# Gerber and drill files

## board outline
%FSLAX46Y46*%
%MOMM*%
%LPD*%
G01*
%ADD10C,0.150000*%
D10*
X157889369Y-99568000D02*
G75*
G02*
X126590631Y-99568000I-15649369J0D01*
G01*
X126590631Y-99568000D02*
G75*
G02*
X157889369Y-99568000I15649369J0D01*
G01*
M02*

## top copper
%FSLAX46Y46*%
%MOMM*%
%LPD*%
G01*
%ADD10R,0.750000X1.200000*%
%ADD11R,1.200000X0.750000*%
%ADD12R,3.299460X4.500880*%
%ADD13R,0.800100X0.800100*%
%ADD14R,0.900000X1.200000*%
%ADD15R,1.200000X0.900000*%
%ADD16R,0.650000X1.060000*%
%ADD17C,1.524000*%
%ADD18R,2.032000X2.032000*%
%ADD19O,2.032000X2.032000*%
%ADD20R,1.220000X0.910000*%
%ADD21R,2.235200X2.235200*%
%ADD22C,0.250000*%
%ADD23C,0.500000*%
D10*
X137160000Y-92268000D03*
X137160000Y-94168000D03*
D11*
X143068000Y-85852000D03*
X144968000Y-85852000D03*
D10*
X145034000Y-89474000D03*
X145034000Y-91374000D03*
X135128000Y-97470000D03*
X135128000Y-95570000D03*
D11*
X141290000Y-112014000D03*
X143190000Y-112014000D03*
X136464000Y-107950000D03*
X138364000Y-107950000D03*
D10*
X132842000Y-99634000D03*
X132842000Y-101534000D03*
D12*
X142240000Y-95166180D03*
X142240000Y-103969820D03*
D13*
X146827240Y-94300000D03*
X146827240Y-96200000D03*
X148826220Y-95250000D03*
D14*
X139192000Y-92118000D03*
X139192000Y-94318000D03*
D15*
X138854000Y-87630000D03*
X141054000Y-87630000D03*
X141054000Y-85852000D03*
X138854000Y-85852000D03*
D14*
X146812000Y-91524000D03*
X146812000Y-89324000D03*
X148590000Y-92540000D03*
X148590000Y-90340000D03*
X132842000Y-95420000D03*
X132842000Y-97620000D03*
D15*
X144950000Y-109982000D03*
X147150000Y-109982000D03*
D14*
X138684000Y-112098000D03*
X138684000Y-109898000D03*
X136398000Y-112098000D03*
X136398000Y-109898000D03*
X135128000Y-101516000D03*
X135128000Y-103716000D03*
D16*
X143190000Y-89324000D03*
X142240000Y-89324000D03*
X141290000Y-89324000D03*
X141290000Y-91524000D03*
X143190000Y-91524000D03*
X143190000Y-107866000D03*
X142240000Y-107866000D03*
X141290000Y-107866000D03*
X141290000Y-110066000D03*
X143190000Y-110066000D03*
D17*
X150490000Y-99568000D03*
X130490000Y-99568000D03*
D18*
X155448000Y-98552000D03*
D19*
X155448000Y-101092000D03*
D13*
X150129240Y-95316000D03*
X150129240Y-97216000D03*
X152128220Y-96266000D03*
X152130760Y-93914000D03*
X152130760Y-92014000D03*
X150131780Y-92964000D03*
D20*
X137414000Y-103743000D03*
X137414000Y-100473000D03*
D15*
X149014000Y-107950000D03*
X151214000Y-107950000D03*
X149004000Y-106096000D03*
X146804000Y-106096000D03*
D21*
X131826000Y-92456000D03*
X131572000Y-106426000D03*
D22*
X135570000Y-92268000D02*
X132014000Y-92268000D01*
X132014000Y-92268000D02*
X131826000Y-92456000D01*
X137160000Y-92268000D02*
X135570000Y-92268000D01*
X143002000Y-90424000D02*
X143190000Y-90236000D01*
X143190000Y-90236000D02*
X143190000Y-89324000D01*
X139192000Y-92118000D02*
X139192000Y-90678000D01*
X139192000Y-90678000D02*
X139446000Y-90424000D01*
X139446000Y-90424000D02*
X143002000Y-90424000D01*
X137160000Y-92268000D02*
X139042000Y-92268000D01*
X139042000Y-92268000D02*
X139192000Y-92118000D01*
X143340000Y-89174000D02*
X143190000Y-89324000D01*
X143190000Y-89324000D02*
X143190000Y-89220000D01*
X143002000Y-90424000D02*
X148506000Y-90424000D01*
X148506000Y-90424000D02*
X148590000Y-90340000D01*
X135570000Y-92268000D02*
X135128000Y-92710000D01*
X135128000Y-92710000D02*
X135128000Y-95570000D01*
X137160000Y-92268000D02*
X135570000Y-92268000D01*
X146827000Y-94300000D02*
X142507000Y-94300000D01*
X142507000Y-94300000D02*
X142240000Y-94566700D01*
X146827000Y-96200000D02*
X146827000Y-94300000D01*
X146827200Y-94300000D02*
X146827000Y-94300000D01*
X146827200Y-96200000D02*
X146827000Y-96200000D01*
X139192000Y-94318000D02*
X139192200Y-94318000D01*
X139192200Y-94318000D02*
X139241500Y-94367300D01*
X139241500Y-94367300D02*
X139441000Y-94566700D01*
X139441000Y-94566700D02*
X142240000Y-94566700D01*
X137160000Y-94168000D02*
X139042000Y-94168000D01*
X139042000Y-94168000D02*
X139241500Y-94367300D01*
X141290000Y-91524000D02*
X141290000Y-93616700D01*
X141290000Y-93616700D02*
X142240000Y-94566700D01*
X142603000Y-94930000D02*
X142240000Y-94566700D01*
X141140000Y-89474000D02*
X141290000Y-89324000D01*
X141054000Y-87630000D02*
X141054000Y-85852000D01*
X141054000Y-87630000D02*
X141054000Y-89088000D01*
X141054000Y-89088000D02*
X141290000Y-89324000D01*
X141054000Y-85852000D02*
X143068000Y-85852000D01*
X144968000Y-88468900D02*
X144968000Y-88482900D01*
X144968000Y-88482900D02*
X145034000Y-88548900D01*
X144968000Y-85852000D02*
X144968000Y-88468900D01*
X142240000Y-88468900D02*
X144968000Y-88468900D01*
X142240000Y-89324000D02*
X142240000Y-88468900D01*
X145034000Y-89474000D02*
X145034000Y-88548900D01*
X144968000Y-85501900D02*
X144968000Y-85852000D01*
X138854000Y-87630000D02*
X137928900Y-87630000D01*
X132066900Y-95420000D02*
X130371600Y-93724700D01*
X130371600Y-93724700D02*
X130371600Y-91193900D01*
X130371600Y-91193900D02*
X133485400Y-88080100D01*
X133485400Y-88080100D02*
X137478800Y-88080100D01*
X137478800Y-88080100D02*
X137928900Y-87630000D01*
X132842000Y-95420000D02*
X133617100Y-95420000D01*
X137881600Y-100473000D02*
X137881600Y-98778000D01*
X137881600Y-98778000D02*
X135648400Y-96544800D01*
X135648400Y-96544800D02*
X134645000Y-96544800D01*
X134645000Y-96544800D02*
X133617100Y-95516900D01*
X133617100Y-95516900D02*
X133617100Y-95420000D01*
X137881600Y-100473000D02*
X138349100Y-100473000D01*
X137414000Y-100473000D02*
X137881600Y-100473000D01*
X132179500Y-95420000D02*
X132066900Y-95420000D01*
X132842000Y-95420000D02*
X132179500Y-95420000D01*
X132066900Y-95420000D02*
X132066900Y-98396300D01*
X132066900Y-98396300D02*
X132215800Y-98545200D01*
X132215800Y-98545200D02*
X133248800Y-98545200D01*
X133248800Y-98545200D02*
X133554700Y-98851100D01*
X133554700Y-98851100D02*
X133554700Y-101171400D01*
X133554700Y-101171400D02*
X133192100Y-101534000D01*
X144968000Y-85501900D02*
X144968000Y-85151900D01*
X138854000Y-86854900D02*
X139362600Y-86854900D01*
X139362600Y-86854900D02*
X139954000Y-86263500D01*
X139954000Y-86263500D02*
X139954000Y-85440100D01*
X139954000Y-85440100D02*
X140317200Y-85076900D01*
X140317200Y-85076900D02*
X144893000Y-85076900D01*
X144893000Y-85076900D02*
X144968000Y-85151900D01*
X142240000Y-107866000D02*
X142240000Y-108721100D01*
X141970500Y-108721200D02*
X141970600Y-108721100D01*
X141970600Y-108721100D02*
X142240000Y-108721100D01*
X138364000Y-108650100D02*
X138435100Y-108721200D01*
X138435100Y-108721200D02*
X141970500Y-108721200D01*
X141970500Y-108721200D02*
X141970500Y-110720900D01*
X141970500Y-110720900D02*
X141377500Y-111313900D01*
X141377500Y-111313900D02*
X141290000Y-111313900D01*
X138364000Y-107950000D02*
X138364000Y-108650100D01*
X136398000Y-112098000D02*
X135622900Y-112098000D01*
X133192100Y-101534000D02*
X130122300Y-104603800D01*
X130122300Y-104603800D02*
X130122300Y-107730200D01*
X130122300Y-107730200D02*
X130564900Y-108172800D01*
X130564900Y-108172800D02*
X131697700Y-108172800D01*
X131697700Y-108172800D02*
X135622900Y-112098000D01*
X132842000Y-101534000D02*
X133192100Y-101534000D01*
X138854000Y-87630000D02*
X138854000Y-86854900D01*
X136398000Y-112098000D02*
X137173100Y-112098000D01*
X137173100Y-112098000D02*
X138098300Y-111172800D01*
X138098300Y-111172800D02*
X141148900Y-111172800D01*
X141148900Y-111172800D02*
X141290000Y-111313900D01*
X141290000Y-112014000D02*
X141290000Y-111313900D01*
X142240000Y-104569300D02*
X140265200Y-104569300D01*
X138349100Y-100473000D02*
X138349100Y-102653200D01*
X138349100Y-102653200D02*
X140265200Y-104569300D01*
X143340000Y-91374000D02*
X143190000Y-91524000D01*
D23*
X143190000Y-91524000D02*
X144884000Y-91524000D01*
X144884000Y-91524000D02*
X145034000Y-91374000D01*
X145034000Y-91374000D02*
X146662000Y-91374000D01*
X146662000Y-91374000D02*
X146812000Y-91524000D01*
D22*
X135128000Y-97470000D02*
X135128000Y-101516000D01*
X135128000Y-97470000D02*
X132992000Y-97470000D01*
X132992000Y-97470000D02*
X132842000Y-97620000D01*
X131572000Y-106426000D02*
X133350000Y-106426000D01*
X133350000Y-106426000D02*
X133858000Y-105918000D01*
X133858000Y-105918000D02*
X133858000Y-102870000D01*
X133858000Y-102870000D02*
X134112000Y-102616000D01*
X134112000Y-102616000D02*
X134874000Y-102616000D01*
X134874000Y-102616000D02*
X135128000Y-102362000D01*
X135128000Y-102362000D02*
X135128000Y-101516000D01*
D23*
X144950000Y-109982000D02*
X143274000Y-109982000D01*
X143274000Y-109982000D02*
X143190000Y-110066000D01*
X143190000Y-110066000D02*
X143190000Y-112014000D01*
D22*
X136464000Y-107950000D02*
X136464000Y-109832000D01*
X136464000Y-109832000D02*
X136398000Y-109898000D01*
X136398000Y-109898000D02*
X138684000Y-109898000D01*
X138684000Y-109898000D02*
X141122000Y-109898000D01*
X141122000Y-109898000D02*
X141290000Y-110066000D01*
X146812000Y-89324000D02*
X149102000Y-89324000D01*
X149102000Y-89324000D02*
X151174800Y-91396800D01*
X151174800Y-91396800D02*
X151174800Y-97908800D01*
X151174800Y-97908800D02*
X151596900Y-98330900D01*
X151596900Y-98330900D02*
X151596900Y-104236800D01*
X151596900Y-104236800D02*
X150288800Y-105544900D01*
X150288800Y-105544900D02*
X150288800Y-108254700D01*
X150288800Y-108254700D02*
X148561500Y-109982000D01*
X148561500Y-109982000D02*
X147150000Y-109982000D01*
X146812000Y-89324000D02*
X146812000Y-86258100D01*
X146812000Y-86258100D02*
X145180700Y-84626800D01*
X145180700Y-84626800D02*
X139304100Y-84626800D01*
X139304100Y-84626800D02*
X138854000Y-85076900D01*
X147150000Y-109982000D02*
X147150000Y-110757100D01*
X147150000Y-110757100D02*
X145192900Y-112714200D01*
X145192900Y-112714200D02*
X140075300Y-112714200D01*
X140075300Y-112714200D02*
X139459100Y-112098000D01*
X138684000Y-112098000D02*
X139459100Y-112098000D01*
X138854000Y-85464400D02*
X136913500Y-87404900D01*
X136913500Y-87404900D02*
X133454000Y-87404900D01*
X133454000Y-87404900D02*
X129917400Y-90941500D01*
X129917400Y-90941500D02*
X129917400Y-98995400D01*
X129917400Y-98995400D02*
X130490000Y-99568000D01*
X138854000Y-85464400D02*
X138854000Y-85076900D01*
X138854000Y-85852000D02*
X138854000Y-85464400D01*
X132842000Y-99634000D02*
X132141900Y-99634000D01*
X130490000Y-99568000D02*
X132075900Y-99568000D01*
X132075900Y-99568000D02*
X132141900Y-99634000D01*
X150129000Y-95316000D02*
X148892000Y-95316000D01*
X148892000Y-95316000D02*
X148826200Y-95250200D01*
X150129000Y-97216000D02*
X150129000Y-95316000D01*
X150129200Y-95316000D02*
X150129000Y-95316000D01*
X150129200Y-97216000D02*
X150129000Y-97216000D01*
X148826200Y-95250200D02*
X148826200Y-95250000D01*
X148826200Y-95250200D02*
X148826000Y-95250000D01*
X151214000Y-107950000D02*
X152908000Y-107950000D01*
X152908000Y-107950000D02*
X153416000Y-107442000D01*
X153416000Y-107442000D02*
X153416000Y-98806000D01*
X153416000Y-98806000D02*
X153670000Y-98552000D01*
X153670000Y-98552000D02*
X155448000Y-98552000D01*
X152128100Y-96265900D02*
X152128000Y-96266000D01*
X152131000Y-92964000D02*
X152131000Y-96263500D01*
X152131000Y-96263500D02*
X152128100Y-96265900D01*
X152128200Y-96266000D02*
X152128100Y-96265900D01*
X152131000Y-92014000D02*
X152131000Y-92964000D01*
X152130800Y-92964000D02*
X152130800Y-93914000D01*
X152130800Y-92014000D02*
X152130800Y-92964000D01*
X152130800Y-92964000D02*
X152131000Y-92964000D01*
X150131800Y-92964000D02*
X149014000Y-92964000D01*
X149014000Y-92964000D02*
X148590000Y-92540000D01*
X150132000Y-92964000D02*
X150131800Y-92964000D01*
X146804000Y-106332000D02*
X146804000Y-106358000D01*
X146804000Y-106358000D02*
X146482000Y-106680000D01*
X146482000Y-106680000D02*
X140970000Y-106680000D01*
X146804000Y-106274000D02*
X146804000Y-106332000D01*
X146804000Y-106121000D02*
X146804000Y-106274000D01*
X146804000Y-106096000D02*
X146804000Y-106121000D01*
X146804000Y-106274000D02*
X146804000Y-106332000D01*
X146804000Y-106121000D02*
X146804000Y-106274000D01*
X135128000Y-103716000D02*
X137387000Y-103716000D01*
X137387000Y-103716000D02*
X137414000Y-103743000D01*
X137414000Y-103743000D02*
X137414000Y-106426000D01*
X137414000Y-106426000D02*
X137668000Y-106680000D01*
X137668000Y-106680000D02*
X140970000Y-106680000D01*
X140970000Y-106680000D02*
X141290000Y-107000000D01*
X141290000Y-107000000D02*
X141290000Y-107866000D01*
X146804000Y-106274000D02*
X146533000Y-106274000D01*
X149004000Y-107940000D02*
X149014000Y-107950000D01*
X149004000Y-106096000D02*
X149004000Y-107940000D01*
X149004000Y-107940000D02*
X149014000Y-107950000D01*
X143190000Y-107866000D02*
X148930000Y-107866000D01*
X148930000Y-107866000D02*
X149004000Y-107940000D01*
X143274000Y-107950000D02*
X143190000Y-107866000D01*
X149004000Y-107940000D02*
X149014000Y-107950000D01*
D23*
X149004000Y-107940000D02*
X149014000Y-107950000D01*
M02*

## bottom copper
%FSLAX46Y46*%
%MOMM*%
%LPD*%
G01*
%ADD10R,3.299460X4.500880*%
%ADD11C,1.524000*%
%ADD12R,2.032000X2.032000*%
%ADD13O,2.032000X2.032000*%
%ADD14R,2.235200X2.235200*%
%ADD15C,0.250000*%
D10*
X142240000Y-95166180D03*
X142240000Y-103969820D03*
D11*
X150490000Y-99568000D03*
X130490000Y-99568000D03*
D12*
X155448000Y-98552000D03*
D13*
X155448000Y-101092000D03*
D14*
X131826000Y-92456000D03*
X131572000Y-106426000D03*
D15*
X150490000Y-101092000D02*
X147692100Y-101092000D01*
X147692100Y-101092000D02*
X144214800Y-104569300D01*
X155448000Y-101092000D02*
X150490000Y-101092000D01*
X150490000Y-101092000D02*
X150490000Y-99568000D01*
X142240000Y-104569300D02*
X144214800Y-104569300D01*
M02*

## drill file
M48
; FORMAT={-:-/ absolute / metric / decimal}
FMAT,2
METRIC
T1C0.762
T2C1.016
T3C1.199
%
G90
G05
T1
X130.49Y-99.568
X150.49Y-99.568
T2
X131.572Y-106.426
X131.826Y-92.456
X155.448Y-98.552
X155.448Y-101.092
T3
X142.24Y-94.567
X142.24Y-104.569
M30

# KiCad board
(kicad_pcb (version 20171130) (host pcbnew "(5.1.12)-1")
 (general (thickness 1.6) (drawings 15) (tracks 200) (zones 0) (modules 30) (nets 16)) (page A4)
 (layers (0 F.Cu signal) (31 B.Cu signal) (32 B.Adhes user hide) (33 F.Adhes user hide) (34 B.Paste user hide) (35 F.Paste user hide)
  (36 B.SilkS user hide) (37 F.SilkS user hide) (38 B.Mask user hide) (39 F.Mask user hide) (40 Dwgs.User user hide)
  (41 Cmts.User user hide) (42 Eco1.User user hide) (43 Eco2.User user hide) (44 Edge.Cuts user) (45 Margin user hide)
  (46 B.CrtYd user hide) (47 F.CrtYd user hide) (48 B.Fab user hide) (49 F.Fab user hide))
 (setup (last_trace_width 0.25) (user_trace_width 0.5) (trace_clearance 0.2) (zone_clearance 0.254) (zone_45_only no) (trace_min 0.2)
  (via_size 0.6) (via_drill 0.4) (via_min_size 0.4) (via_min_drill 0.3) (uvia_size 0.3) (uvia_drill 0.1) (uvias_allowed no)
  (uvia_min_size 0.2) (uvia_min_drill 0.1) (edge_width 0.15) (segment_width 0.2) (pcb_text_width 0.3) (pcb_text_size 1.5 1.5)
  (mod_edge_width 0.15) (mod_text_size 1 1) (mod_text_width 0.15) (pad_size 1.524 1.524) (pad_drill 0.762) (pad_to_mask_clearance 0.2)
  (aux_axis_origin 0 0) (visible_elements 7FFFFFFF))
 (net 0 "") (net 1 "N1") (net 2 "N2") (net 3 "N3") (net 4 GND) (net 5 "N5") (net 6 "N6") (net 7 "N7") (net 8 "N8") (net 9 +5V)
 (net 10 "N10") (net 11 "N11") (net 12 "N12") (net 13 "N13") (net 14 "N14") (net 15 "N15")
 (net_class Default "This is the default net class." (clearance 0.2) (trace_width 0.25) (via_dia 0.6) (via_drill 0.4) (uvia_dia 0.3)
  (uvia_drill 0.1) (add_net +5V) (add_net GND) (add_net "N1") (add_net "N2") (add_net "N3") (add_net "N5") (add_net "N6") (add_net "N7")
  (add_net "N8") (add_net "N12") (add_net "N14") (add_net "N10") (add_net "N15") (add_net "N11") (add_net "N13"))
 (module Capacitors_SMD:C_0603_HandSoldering (layer F.Cu) (at 137.16 93.218 270)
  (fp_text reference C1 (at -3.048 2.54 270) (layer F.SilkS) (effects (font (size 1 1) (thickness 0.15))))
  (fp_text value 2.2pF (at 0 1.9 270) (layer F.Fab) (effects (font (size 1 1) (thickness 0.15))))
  (pad 1 smd rect (at -0.95 0 270) (size 1.2 0.75) (layers F.Cu F.Paste F.Mask) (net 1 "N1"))
  (pad 2 smd rect (at 0.95 0 270) (size 1.2 0.75) (layers F.Cu F.Paste F.Mask) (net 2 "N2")))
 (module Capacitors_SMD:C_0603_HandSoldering (layer F.Cu) (at 144.018 85.852)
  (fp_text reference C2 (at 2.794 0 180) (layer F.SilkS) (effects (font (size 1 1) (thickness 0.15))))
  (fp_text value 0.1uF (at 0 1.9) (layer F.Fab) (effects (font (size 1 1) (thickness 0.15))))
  (pad 1 smd rect (at -0.95 0) (size 1.2 0.75) (layers F.Cu F.Paste F.Mask) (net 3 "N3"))
  (pad 2 smd rect (at 0.95 0) (size 1.2 0.75) (layers F.Cu F.Paste F.Mask) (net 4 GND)))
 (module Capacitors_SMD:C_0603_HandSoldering (layer F.Cu) (at 145.034 90.424 270)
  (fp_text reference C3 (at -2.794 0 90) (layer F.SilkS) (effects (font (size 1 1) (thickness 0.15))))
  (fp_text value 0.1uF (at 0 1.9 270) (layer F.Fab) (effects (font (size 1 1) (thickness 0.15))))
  (pad 1 smd rect (at -0.95 0 270) (size 1.2 0.75) (layers F.Cu F.Paste F.Mask) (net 4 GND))
  (pad 2 smd rect (at 0.95 0 270) (size 1.2 0.75) (layers F.Cu F.Paste F.Mask) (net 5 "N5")))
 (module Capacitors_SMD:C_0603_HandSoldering (layer F.Cu) (at 135.128 96.52 90)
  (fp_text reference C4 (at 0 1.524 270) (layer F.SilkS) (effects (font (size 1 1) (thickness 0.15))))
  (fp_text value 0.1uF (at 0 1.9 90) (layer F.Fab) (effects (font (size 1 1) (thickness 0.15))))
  (pad 1 smd rect (at -0.95 0 90) (size 1.2 0.75) (layers F.Cu F.Paste F.Mask) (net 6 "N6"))
  (pad 2 smd rect (at 0.95 0 90) (size 1.2 0.75) (layers F.Cu F.Paste F.Mask) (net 1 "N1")))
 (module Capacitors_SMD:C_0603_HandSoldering (layer F.Cu) (at 142.24 112.014)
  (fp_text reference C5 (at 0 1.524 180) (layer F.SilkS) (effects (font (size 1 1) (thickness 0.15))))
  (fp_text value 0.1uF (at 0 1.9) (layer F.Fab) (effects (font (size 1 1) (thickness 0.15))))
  (pad 1 smd rect (at -0.95 0) (size 1.2 0.75) (layers F.Cu F.Paste F.Mask) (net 4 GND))
  (pad 2 smd rect (at 0.95 0) (size 1.2 0.75) (layers F.Cu F.Paste F.Mask) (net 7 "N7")))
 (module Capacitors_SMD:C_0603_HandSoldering (layer F.Cu) (at 137.414 107.95)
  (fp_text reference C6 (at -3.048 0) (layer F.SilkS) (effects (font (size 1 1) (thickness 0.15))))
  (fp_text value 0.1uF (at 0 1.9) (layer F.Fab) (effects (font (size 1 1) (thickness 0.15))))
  (pad 1 smd rect (at -0.95 0) (size 1.2 0.75) (layers F.Cu F.Paste F.Mask) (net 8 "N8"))
  (pad 2 smd rect (at 0.95 0) (size 1.2 0.75) (layers F.Cu F.Paste F.Mask) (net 4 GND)))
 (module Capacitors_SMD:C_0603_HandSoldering (layer F.Cu) (at 132.842 100.584 270)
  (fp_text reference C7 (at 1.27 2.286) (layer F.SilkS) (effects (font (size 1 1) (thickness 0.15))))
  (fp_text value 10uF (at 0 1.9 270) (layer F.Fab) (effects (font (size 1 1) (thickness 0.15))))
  (pad 1 smd rect (at -0.95 0 270) (size 1.2 0.75) (layers F.Cu F.Paste F.Mask) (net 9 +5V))
  (pad 2 smd rect (at 0.95 0 270) (size 1.2 0.75) (layers F.Cu F.Paste F.Mask) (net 4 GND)))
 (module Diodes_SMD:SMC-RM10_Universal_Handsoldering (layer F.Cu) (at 142.24 99.568 270)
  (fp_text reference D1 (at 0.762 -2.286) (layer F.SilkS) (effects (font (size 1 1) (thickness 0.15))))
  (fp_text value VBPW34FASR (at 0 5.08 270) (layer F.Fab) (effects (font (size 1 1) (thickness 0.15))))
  (pad 1 thru_hole rect (at -5.00126 0 270) (size 4.50088 3.29946) (drill 1.19888 (offset 0.59944 0)) (layers *.Cu *.Mask F.SilkS)
   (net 2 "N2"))
  (pad 2 thru_hole rect (at 5.00126 0 90) (size 4.50088 3.29946) (drill 1.19888 (offset 0.59944 0)) (layers *.Cu *.Mask F.SilkS) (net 4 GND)))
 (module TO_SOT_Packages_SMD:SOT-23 (layer F.Cu) (at 147.828 95.25 270)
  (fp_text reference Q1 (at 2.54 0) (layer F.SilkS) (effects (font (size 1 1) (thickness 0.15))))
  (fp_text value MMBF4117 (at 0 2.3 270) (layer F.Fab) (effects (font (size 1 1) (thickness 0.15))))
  (pad 1 smd rect (at -0.95 1.00076 270) (size 0.8001 0.8001) (layers F.Cu F.Paste F.Mask) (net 2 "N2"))
  (pad 2 smd rect (at 0.95 1.00076 270) (size 0.8001 0.8001) (layers F.Cu F.Paste F.Mask) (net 2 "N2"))
  (pad 3 smd rect (at 0 -0.99822 270) (size 0.8001 0.8001) (layers F.Cu F.Paste F.Mask) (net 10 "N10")))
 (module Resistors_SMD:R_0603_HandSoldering (layer F.Cu) (at 139.192 93.218 270)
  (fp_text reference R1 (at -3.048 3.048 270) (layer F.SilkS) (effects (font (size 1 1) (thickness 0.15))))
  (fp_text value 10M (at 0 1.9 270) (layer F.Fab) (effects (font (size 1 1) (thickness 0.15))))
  (pad 1 smd rect (at -1.1 0 270) (size 1.2 0.9) (layers F.Cu F.Paste F.Mask) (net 1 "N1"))
  (pad 2 smd rect (at 1.1 0 270) (size 1.2 0.9) (layers F.Cu F.Paste F.Mask) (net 2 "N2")))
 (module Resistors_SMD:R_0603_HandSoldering (layer F.Cu) (at 139.954 87.63)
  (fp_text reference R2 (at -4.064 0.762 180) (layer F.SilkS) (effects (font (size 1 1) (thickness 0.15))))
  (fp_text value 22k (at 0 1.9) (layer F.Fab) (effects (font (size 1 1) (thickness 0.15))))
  (pad 1 smd rect (at -1.1 0) (size 1.2 0.9) (layers F.Cu F.Paste F.Mask) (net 4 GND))
  (pad 2 smd rect (at 1.1 0) (size 1.2 0.9) (layers F.Cu F.Paste F.Mask) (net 3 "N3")))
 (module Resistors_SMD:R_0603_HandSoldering (layer F.Cu) (at 139.954 85.852 180)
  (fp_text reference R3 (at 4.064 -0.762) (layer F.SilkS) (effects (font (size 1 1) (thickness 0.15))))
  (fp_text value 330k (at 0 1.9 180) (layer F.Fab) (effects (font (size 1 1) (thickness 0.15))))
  (pad 1 smd rect (at -1.1 0 180) (size 1.2 0.9) (layers F.Cu F.Paste F.Mask) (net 3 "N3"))
  (pad 2 smd rect (at 1.1 0 180) (size 1.2 0.9) (layers F.Cu F.Paste F.Mask) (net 9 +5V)))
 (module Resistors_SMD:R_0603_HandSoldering (layer F.Cu) (at 146.812 90.424 90)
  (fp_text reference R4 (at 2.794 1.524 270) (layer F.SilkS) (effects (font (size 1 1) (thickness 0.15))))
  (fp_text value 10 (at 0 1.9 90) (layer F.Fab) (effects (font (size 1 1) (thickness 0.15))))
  (pad 1 smd rect (at -1.1 0 90) (size 1.2 0.9) (layers F.Cu F.Paste F.Mask) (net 5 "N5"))
  (pad 2 smd rect (at 1.1 0 90) (size 1.2 0.9) (layers F.Cu F.Paste F.Mask) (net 9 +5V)))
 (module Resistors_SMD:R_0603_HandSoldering (layer F.Cu) (at 148.59 91.44 90)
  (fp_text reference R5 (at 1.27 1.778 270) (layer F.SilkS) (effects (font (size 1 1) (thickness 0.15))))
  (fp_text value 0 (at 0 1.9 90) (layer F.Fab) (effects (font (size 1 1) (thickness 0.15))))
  (pad 1 smd rect (at -1.1 0 90) (size 1.2 0.9) (layers F.Cu F.Paste F.Mask) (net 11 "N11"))
  (pad 2 smd rect (at 1.1 0 90) (size 1.2 0.9) (layers F.Cu F.Paste F.Mask) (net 1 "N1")))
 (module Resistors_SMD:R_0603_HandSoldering (layer F.Cu) (at 132.842 96.52 270)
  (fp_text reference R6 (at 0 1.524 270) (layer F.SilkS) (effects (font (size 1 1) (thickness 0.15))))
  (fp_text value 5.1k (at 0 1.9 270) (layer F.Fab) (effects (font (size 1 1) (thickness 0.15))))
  (pad 1 smd rect (at -1.1 0 270) (size 1.2 0.9) (layers F.Cu F.Paste F.Mask) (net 4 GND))
  (pad 2 smd rect (at 1.1 0 270) (size 1.2 0.9) (layers F.Cu F.Paste F.Mask) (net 6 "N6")))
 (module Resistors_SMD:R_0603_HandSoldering (layer F.Cu) (at 146.05 109.982)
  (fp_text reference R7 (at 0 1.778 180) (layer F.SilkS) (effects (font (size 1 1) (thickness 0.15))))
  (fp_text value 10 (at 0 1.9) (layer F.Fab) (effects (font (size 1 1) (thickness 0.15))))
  (pad 1 smd rect (at -1.1 0) (size 1.2 0.9) (layers F.Cu F.Paste F.Mask) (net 7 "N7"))
  (pad 2 smd rect (at 1.1 0) (size 1.2 0.9) (layers F.Cu F.Paste F.Mask) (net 9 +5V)))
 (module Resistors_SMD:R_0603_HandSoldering (layer F.Cu) (at 138.684 110.998 90)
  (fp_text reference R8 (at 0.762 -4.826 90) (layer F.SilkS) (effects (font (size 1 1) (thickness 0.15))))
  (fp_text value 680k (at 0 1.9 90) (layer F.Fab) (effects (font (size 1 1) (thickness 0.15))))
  (pad 1 smd rect (at -1.1 0 90) (size 1.2 0.9) (layers F.Cu F.Paste F.Mask) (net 9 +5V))
  (pad 2 smd rect (at 1.1 0 90) (size 1.2 0.9) (layers F.Cu F.Paste F.Mask) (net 8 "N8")))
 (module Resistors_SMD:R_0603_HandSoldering (layer F.Cu) (at 136.398 110.998 90)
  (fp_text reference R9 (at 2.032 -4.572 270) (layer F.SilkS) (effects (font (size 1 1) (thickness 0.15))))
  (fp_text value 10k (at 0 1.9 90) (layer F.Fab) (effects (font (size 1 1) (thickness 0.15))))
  (pad 1 smd rect (at -1.1 0 90) (size 1.2 0.9) (layers F.Cu F.Paste F.Mask) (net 4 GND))
  (pad 2 smd rect (at 1.1 0 90) (size 1.2 0.9) (layers F.Cu F.Paste F.Mask) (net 8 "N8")))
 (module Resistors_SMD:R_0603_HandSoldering (layer F.Cu) (at 135.128 102.616 270)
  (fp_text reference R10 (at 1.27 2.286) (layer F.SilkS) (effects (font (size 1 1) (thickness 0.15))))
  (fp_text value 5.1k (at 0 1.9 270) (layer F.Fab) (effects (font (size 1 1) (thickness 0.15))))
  (pad 1 smd rect (at -1.1 0 270) (size 1.2 0.9) (layers F.Cu F.Paste F.Mask) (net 6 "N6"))
  (pad 2 smd rect (at 1.1 0 270) (size 1.2 0.9) (layers F.Cu F.Paste F.Mask) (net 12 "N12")))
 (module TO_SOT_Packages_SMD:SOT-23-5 (layer F.Cu) (at 142.24 90.424 270)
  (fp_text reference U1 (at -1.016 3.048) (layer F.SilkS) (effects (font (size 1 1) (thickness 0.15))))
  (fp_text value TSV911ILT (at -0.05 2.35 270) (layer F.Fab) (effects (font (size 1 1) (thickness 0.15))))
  (pad 1 smd rect (at -1.1 -0.95 270) (size 1.06 0.65) (layers F.Cu F.Paste F.Mask) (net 1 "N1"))
  (pad 2 smd rect (at -1.1 0 270) (size 1.06 0.65) (layers F.Cu F.Paste F.Mask) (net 4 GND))
  (pad 3 smd rect (at -1.1 0.95 270) (size 1.06 0.65) (layers F.Cu F.Paste F.Mask) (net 3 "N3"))
  (pad 4 smd rect (at 1.1 0.95 270) (size 1.06 0.65) (layers F.Cu F.Paste F.Mask) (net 2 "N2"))
  (pad 5 smd rect (at 1.1 -0.95 270) (size 1.06 0.65) (layers F.Cu F.Paste F.Mask) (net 5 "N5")))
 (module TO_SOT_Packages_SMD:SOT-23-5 (layer F.Cu) (at 142.24 108.966 270)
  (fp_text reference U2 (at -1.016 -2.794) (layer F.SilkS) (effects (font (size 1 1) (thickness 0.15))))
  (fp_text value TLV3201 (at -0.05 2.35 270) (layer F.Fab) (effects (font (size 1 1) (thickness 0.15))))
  (pad 1 smd rect (at -1.1 -0.95 270) (size 1.06 0.65) (layers F.Cu F.Paste F.Mask) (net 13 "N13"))
  (pad 2 smd rect (at -1.1 0 270) (size 1.06 0.65) (layers F.Cu F.Paste F.Mask) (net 4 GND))
  (pad 3 smd rect (at -1.1 0.95 270) (size 1.06 0.65) (layers F.Cu F.Paste F.Mask) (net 12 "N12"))
  (pad 4 smd rect (at 1.1 0.95 270) (size 1.06 0.65) (layers F.Cu F.Paste F.Mask) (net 8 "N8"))
  (pad 5 smd rect (at 1.1 -0.95 270) (size 1.06 0.65) (layers F.Cu F.Paste F.Mask) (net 7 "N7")))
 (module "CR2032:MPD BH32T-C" (layer B.Cu) (at 142.24 99.568 90)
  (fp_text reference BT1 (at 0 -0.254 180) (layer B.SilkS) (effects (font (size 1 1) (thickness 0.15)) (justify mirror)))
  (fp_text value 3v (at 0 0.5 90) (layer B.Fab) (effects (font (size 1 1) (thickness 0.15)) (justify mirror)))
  (pad 2 thru_hole circle (at 0 8.25 90) (size 1.524 1.524) (drill 0.762) (layers *.Cu *.Mask B.SilkS) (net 4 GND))
  (pad 1 thru_hole circle (at 0 -11.75 90) (size 1.524 1.524) (drill 0.762) (layers *.Cu *.Mask B.SilkS) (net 9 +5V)))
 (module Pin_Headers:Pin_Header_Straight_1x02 (layer F.Cu) (at 155.448 98.552)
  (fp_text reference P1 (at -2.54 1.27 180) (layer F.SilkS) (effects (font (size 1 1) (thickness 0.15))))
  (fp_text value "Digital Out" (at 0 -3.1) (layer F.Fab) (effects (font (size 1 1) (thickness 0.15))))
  (pad 1 thru_hole rect (at 0 0) (size 2.032 2.032) (drill 1.016) (layers *.Cu *.Mask F.SilkS) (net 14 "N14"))
  (pad 2 thru_hole oval (at 0 2.54) (size 2.032 2.032) (drill 1.016) (layers *.Cu *.Mask F.SilkS) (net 4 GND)))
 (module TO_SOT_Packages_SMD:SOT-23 (layer F.Cu) (at 151.13 96.266 270)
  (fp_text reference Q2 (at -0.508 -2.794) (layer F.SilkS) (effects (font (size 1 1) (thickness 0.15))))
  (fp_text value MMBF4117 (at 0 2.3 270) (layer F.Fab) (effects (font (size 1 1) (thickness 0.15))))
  (pad 1 smd rect (at -0.95 1.00076 270) (size 0.8001 0.8001) (layers F.Cu F.Paste F.Mask) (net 10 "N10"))
  (pad 2 smd rect (at 0.95 1.00076 270) (size 0.8001 0.8001) (layers F.Cu F.Paste F.Mask) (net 10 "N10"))
  (pad 3 smd rect (at 0 -0.99822 270) (size 0.8001 0.8001) (layers F.Cu F.Paste F.Mask) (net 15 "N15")))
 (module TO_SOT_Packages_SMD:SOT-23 (layer F.Cu) (at 151.13 92.964 90)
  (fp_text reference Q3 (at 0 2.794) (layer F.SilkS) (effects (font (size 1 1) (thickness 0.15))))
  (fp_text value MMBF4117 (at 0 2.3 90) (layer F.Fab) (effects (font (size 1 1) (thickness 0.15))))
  (pad 1 smd rect (at -0.95 1.00076 90) (size 0.8001 0.8001) (layers F.Cu F.Paste F.Mask) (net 15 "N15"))
  (pad 2 smd rect (at 0.95 1.00076 90) (size 0.8001 0.8001) (layers F.Cu F.Paste F.Mask) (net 15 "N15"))
  (pad 3 smd rect (at 0 -0.99822 90) (size 0.8001 0.8001) (layers F.Cu F.Paste F.Mask) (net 11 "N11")))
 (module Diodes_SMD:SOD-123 (layer F.Cu) (at 137.414 102.108 90)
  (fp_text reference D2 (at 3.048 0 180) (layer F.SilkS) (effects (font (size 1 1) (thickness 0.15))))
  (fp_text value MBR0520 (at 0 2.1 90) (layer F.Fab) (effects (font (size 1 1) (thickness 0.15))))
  (pad 1 smd rect (at -1.635 0 90) (size 0.91 1.22) (layers F.Cu F.Paste F.Mask) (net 12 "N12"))
  (pad 2 smd rect (at 1.635 0 90) (size 0.91 1.22) (layers F.Cu F.Paste F.Mask) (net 4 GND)))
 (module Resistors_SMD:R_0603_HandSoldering (layer F.Cu) (at 150.114 107.95)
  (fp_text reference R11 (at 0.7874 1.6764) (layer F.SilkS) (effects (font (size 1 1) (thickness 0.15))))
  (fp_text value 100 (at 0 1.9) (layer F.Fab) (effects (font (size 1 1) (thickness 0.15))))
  (pad 1 smd rect (at -1.1 0) (size 1.2 0.9) (layers F.Cu F.Paste F.Mask) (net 13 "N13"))
  (pad 2 smd rect (at 1.1 0) (size 1.2 0.9) (layers F.Cu F.Paste F.Mask) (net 14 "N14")))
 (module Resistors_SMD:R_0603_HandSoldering (layer F.Cu) (at 147.904 106.096 180)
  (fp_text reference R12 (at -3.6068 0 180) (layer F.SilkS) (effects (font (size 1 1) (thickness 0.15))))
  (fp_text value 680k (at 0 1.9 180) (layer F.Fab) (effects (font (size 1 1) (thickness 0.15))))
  (pad 1 smd rect (at -1.1 0 180) (size 1.2 0.9) (layers F.Cu F.Paste F.Mask) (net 13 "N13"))
  (pad 2 smd rect (at 1.1 0 180) (size 1.2 0.9) (layers F.Cu F.Paste F.Mask) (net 12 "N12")))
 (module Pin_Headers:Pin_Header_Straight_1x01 (layer F.Cu) (at 131.826 92.456)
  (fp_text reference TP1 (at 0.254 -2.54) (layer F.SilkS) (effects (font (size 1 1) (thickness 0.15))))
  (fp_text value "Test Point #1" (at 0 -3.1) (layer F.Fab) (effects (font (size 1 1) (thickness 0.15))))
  (pad 1 thru_hole rect (at 0 0) (size 2.2352 2.2352) (drill 1.016) (layers *.Cu *.Mask F.SilkS) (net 1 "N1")))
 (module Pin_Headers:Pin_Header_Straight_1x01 (layer F.Cu) (at 131.572 106.426)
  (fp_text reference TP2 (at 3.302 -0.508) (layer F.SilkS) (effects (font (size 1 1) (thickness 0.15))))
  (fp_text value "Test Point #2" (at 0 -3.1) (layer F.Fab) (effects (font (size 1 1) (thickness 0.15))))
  (pad 1 thru_hole rect (at 0 0) (size 2.2352 2.2352) (drill 1.016) (layers *.Cu *.Mask F.SilkS) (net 6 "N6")))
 (gr_circle (center 142.24 99.568) (end 154.94 108.712) (layer Edge.Cuts) (width 0.15))
 (segment (start 135.57 92.268) (end 132.014 92.268) (width 0.25) (layer F.Cu) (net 1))
 (segment (start 132.014 92.268) (end 131.826 92.456) (width 0.25) (layer F.Cu) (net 1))
 (segment (start 137.16 92.268) (end 135.57 92.268) (width 0.25) (layer F.Cu) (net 1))
 (segment (start 143.002 90.424) (end 143.19 90.236) (width 0.25) (layer F.Cu) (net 1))
 (segment (start 143.19 90.236) (end 143.19 89.324) (width 0.25) (layer F.Cu) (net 1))
 (segment (start 139.192 92.118) (end 139.192 90.678) (width 0.25) (layer F.Cu) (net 1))
 (segment (start 139.192 90.678) (end 139.446 90.424) (width 0.25) (layer F.Cu) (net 1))
 (segment (start 139.446 90.424) (end 143.002 90.424) (width 0.25) (layer F.Cu) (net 1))
 (segment (start 137.16 92.268) (end 139.042 92.268) (width 0.25) (layer F.Cu) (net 1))
 (segment (start 139.042 92.268) (end 139.192 92.118) (width 0.25) (layer F.Cu) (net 1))
 (segment (start 143.34 89.174) (end 143.19 89.324) (width 0.25) (layer F.Cu) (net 1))
 (segment (start 143.19 89.324) (end 143.19 89.22) (width 0.25) (layer F.Cu) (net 1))
 (segment (start 143.002 90.424) (end 148.506 90.424) (width 0.25) (layer F.Cu) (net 1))
 (segment (start 148.506 90.424) (end 148.59 90.34) (width 0.25) (layer F.Cu) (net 1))
 (segment (start 135.57 92.268) (end 135.128 92.71) (width 0.25) (layer F.Cu) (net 1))
 (segment (start 135.128 92.71) (end 135.128 95.57) (width 0.25) (layer F.Cu) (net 1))
 (segment (start 137.16 92.268) (end 135.57 92.268) (width 0.25) (layer F.Cu) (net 1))
 (segment (start 146.827 94.3) (end 142.507 94.3) (width 0.25) (layer F.Cu) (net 2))
 (segment (start 142.507 94.3) (end 142.24 94.5667) (width 0.25) (layer F.Cu) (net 2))
 (segment (start 146.827 96.2) (end 146.827 94.3) (width 0.25) (layer F.Cu) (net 2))
 (segment (start 146.8272 94.3) (end 146.827 94.3) (width 0.25) (layer F.Cu) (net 2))
 (segment (start 146.8272 96.2) (end 146.827 96.2) (width 0.25) (layer F.Cu) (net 2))
 (segment (start 139.192 94.318) (end 139.1922 94.318) (width 0.25) (layer F.Cu) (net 2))
 (segment (start 139.1922 94.318) (end 139.2415 94.3673) (width 0.25) (layer F.Cu) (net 2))
 (segment (start 139.2415 94.3673) (end 139.441 94.5667) (width 0.25) (layer F.Cu) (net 2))
 (segment (start 139.441 94.5667) (end 142.24 94.5667) (width 0.25) (layer F.Cu) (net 2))
 (segment (start 137.16 94.168) (end 139.042 94.168) (width 0.25) (layer F.Cu) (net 2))
 (segment (start 139.042 94.168) (end 139.2415 94.3673) (width 0.25) (layer F.Cu) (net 2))
 (segment (start 141.29 91.524) (end 141.29 93.6167) (width 0.25) (layer F.Cu) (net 2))
 (segment (start 141.29 93.6167) (end 142.24 94.5667) (width 0.25) (layer F.Cu) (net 2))
 (segment (start 142.603 94.93) (end 142.24 94.5667) (width 0.25) (layer F.Cu) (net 2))
 (segment (start 141.14 89.474) (end 141.29 89.324) (width 0.25) (layer F.Cu) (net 3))
 (segment (start 141.054 87.63) (end 141.054 85.852) (width 0.25) (layer F.Cu) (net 3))
 (segment (start 141.054 87.63) (end 141.054 89.088) (width 0.25) (layer F.Cu) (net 3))
 (segment (start 141.054 89.088) (end 141.29 89.324) (width 0.25) (layer F.Cu) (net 3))
 (segment (start 141.054 85.852) (end 143.068 85.852) (width 0.25) (layer F.Cu) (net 3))
 (segment (start 144.968 88.4689) (end 144.968 88.4829) (width 0.25) (layer F.Cu) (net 4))
 (segment (start 144.968 88.4829) (end 145.034 88.5489) (width 0.25) (layer F.Cu) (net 4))
 (segment (start 144.968 85.852) (end 144.968 88.4689) (width 0.25) (layer F.Cu) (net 4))
 (segment (start 142.24 88.4689) (end 144.968 88.4689) (width 0.25) (layer F.Cu) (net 4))
 (segment (start 142.24 89.324) (end 142.24 88.4689) (width 0.25) (layer F.Cu) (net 4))
 (segment (start 145.034 89.474) (end 145.034 88.5489) (width 0.25) (layer F.Cu) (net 4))
 (segment (start 144.968 85.5019) (end 144.968 85.852) (width 0.25) (layer F.Cu) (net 4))
 (segment (start 138.854 87.63) (end 137.9289 87.63) (width 0.25) (layer F.Cu) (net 4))
 (segment (start 132.0669 95.42) (end 130.3716 93.7247) (width 0.25) (layer F.Cu) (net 4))
 (segment (start 130.3716 93.7247) (end 130.3716 91.1939) (width 0.25) (layer F.Cu) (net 4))
 (segment (start 130.3716 91.1939) (end 133.4854 88.0801) (width 0.25) (layer F.Cu) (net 4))
 (segment (start 133.4854 88.0801) (end 137.4788 88.0801) (width 0.25) (layer F.Cu) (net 4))
 (segment (start 137.4788 88.0801) (end 137.9289 87.63) (width 0.25) (layer F.Cu) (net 4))
 (segment (start 132.842 95.42) (end 133.6171 95.42) (width 0.25) (layer F.Cu) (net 4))
 (segment (start 137.8816 100.473) (end 137.8816 98.778) (width 0.25) (layer F.Cu) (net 4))
 (segment (start 137.8816 98.778) (end 135.6484 96.5448) (width 0.25) (layer F.Cu) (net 4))
 (segment (start 135.6484 96.5448) (end 134.645 96.5448) (width 0.25) (layer F.Cu) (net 4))
 (segment (start 134.645 96.5448) (end 133.6171 95.5169) (width 0.25) (layer F.Cu) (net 4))
 (segment (start 133.6171 95.5169) (end 133.6171 95.42) (width 0.25) (layer F.Cu) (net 4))
 (segment (start 137.8816 100.473) (end 138.3491 100.473) (width 0.25) (layer F.Cu) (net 4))
 (segment (start 137.414 100.473) (end 137.8816 100.473) (width 0.25) (layer F.Cu) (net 4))
 (segment (start 132.1795 95.42) (end 132.0669 95.42) (width 0.25) (layer F.Cu) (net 4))
 (segment (start 132.842 95.42) (end 132.1795 95.42) (width 0.25) (layer F.Cu) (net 4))
 (segment (start 132.0669 95.42) (end 132.0669 98.3963) (width 0.25) (layer F.Cu) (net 4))
 (segment (start 132.0669 98.3963) (end 132.2158 98.5452) (width 0.25) (layer F.Cu) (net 4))
 (segment (start 132.2158 98.5452) (end 133.2488 98.5452) (width 0.25) (layer F.Cu) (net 4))
 (segment (start 133.2488 98.5452) (end 133.5547 98.8511) (width 0.25) (layer F.Cu) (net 4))
 (segment (start 133.5547 98.8511) (end 133.5547 101.1714) (width 0.25) (layer F.Cu) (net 4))
 (segment (start 133.5547 101.1714) (end 133.1921 101.534) (width 0.25) (layer F.Cu) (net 4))
 (segment (start 144.968 85.5019) (end 144.968 85.1519) (width 0.25) (layer F.Cu) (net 4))
 (segment (start 138.854 86.8549) (end 139.3626 86.8549) (width 0.25) (layer F.Cu) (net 4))
 (segment (start 139.3626 86.8549) (end 139.954 86.2635) (width 0.25) (layer F.Cu) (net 4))
 (segment (start 139.954 86.2635) (end 139.954 85.4401) (width 0.25) (layer F.Cu) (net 4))
 (segment (start 139.954 85.4401) (end 140.3172 85.0769) (width 0.25) (layer F.Cu) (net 4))
 (segment (start 140.3172 85.0769) (end 144.893 85.0769) (width 0.25) (layer F.Cu) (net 4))
 (segment (start 144.893 85.0769) (end 144.968 85.1519) (width 0.25) (layer F.Cu) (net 4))
 (segment (start 142.24 107.866) (end 142.24 108.7211) (width 0.25) (layer F.Cu) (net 4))
 (segment (start 141.9705 108.7212) (end 141.9706 108.7211) (width 0.25) (layer F.Cu) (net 4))
 (segment (start 141.9706 108.7211) (end 142.24 108.7211) (width 0.25) (layer F.Cu) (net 4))
 (segment (start 138.364 108.6501) (end 138.4351 108.7212) (width 0.25) (layer F.Cu) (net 4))
 (segment (start 138.4351 108.7212) (end 141.9705 108.7212) (width 0.25) (layer F.Cu) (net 4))
 (segment (start 141.9705 108.7212) (end 141.9705 110.7209) (width 0.25) (layer F.Cu) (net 4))
 (segment (start 141.9705 110.7209) (end 141.3775 111.3139) (width 0.25) (layer F.Cu) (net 4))
 (segment (start 141.3775 111.3139) (end 141.29 111.3139) (width 0.25) (layer F.Cu) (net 4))
 (segment (start 138.364 107.95) (end 138.364 108.6501) (width 0.25) (layer F.Cu) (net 4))
 (segment (start 136.398 112.098) (end 135.6229 112.098) (width 0.25) (layer F.Cu) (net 4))
 (segment (start 133.1921 101.534) (end 130.1223 104.6038) (width 0.25) (layer F.Cu) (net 4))
 (segment (start 130.1223 104.6038) (end 130.1223 107.7302) (width 0.25) (layer F.Cu) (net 4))
 (segment (start 130.1223 107.7302) (end 130.5649 108.1728) (width 0.25) (layer F.Cu) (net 4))
 (segment (start 130.5649 108.1728) (end 131.6977 108.1728) (width 0.25) (layer F.Cu) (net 4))
 (segment (start 131.6977 108.1728) (end 135.6229 112.098) (width 0.25) (layer F.Cu) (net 4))
 (segment (start 132.842 101.534) (end 133.1921 101.534) (width 0.25) (layer F.Cu) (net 4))
 (segment (start 138.854 87.63) (end 138.854 86.8549) (width 0.25) (layer F.Cu) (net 4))
 (segment (start 136.398 112.098) (end 137.1731 112.098) (width 0.25) (layer F.Cu) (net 4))
 (segment (start 137.1731 112.098) (end 138.0983 111.1728) (width 0.25) (layer F.Cu) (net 4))
 (segment (start 138.0983 111.1728) (end 141.1489 111.1728) (width 0.25) (layer F.Cu) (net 4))
 (segment (start 141.1489 111.1728) (end 141.29 111.3139) (width 0.25) (layer F.Cu) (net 4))
 (segment (start 141.29 112.014) (end 141.29 111.3139) (width 0.25) (layer F.Cu) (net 4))
 (segment (start 150.49 101.092) (end 147.6921 101.092) (width 0.25) (layer B.Cu) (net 4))
 (segment (start 147.6921 101.092) (end 144.2148 104.5693) (width 0.25) (layer B.Cu) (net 4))
 (segment (start 155.448 101.092) (end 150.49 101.092) (width 0.25) (layer B.Cu) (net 4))
 (segment (start 150.49 101.092) (end 150.49 99.568) (width 0.25) (layer B.Cu) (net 4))
 (segment (start 142.24 104.5693) (end 144.2148 104.5693) (width 0.25) (layer B.Cu) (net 4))
 (segment (start 142.24 104.5693) (end 140.2652 104.5693) (width 0.25) (layer F.Cu) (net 4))
 (segment (start 138.3491 100.473) (end 138.3491 102.6532) (width 0.25) (layer F.Cu) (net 4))
 (segment (start 138.3491 102.6532) (end 140.2652 104.5693) (width 0.25) (layer F.Cu) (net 4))
 (segment (start 143.34 91.374) (end 143.19 91.524) (width 0.25) (layer F.Cu) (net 5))
 (segment (start 143.19 91.524) (end 144.884 91.524) (width 0.5) (layer F.Cu) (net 5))
 (segment (start 144.884 91.524) (end 145.034 91.374) (width 0.5) (layer F.Cu) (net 5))
 (segment (start 145.034 91.374) (end 146.662 91.374) (width 0.5) (layer F.Cu) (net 5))
 (segment (start 146.662 91.374) (end 146.812 91.524) (width 0.5) (layer F.Cu) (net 5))
 (segment (start 135.128 97.47) (end 135.128 101.516) (width 0.25) (layer F.Cu) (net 6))
 (segment (start 135.128 97.47) (end 132.992 97.47) (width 0.25) (layer F.Cu) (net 6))
 (segment (start 132.992 97.47) (end 132.842 97.62) (width 0.25) (layer F.Cu) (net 6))
 (segment (start 131.572 106.426) (end 133.35 106.426) (width 0.25) (layer F.Cu) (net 6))
 (segment (start 133.35 106.426) (end 133.858 105.918) (width 0.25) (layer F.Cu) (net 6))
 (segment (start 133.858 105.918) (end 133.858 102.87) (width 0.25) (layer F.Cu) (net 6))
 (segment (start 133.858 102.87) (end 134.112 102.616) (width 0.25) (layer F.Cu) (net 6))
 (segment (start 134.112 102.616) (end 134.874 102.616) (width 0.25) (layer F.Cu) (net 6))
 (segment (start 134.874 102.616) (end 135.128 102.362) (width 0.25) (layer F.Cu) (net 6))
 (segment (start 135.128 102.362) (end 135.128 101.516) (width 0.25) (layer F.Cu) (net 6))
 (segment (start 144.95 109.982) (end 143.274 109.982) (width 0.5) (layer F.Cu) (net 7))
 (segment (start 143.274 109.982) (end 143.19 110.066) (width 0.5) (layer F.Cu) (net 7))
 (segment (start 143.19 110.066) (end 143.19 112.014) (width 0.5) (layer F.Cu) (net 7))
 (segment (start 136.464 107.95) (end 136.464 109.832) (width 0.25) (layer F.Cu) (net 8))
 (segment (start 136.464 109.832) (end 136.398 109.898) (width 0.25) (layer F.Cu) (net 8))
 (segment (start 136.398 109.898) (end 138.684 109.898) (width 0.25) (layer F.Cu) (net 8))
 (segment (start 138.684 109.898) (end 141.122 109.898) (width 0.25) (layer F.Cu) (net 8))
 (segment (start 141.122 109.898) (end 141.29 110.066) (width 0.25) (layer F.Cu) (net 8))
 (segment (start 146.812 89.324) (end 149.102 89.324) (width 0.25) (layer F.Cu) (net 9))
 (segment (start 149.102 89.324) (end 151.1748 91.3968) (width 0.25) (layer F.Cu) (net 9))
 (segment (start 151.1748 91.3968) (end 151.1748 97.9088) (width 0.25) (layer F.Cu) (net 9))
 (segment (start 151.1748 97.9088) (end 151.5969 98.3309) (width 0.25) (layer F.Cu) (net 9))
 (segment (start 151.5969 98.3309) (end 151.5969 104.2368) (width 0.25) (layer F.Cu) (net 9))
 (segment (start 151.5969 104.2368) (end 150.2888 105.5449) (width 0.25) (layer F.Cu) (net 9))
 (segment (start 150.2888 105.5449) (end 150.2888 108.2547) (width 0.25) (layer F.Cu) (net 9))
 (segment (start 150.2888 108.2547) (end 148.5615 109.982) (width 0.25) (layer F.Cu) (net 9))
 (segment (start 148.5615 109.982) (end 147.15 109.982) (width 0.25) (layer F.Cu) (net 9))
 (segment (start 146.812 89.324) (end 146.812 86.2581) (width 0.25) (layer F.Cu) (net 9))
 (segment (start 146.812 86.2581) (end 145.1807 84.6268) (width 0.25) (layer F.Cu) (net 9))
 (segment (start 145.1807 84.6268) (end 139.3041 84.6268) (width 0.25) (layer F.Cu) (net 9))
 (segment (start 139.3041 84.6268) (end 138.854 85.0769) (width 0.25) (layer F.Cu) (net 9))
 (segment (start 147.15 109.982) (end 147.15 110.7571) (width 0.25) (layer F.Cu) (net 9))
 (segment (start 147.15 110.7571) (end 145.1929 112.7142) (width 0.25) (layer F.Cu) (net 9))
 (segment (start 145.1929 112.7142) (end 140.0753 112.7142) (width 0.25) (layer F.Cu) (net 9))
 (segment (start 140.0753 112.7142) (end 139.4591 112.098) (width 0.25) (layer F.Cu) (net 9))
 (segment (start 138.684 112.098) (end 139.4591 112.098) (width 0.25) (layer F.Cu) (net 9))
 (segment (start 138.854 85.4644) (end 136.9135 87.4049) (width 0.25) (layer F.Cu) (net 9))
 (segment (start 136.9135 87.4049) (end 133.454 87.4049) (width 0.25) (layer F.Cu) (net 9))
 (segment (start 133.454 87.4049) (end 129.9174 90.9415) (width 0.25) (layer F.Cu) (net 9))
 (segment (start 129.9174 90.9415) (end 129.9174 98.9954) (width 0.25) (layer F.Cu) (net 9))
 (segment (start 129.9174 98.9954) (end 130.49 99.568) (width 0.25) (layer F.Cu) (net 9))
 (segment (start 138.854 85.4644) (end 138.854 85.0769) (width 0.25) (layer F.Cu) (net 9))
 (segment (start 138.854 85.852) (end 138.854 85.4644) (width 0.25) (layer F.Cu) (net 9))
 (segment (start 132.842 99.634) (end 132.1419 99.634) (width 0.25) (layer F.Cu) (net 9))
 (segment (start 130.49 99.568) (end 132.0759 99.568) (width 0.25) (layer F.Cu) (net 9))
 (segment (start 132.0759 99.568) (end 132.1419 99.634) (width 0.25) (layer F.Cu) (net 9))
 (segment (start 150.129 95.316) (end 148.892 95.316) (width 0.25) (layer F.Cu) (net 10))
 (segment (start 148.892 95.316) (end 148.8262 95.2502) (width 0.25) (layer F.Cu) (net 10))
 (segment (start 150.129 97.216) (end 150.129 95.316) (width 0.25) (layer F.Cu) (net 10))
 (segment (start 150.1292 95.316) (end 150.129 95.316) (width 0.25) (layer F.Cu) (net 10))
 (segment (start 150.1292 97.216) (end 150.129 97.216) (width 0.25) (layer F.Cu) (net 10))
 (segment (start 148.8262 95.2502) (end 148.8262 95.25) (width 0.25) (layer F.Cu) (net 10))
 (segment (start 148.8262 95.2502) (end 148.826 95.25) (width 0.25) (layer F.Cu) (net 10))
 (segment (start 151.214 107.95) (end 152.908 107.95) (width 0.25) (layer F.Cu) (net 14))
 (segment (start 152.908 107.95) (end 153.416 107.442) (width 0.25) (layer F.Cu) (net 14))
 (segment (start 153.416 107.442) (end 153.416 98.806) (width 0.25) (layer F.Cu) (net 14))
 (segment (start 153.416 98.806) (end 153.67 98.552) (width 0.25) (layer F.Cu) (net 14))
 (segment (start 153.67 98.552) (end 155.448 98.552) (width 0.25) (layer F.Cu) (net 14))
 (segment (start 152.1281 96.2659) (end 152.128 96.266) (width 0.25) (layer F.Cu) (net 15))
 (segment (start 152.131 92.964) (end 152.131 96.2635) (width 0.25) (layer F.Cu) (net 15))
 (segment (start 152.131 96.2635) (end 152.1281 96.2659) (width 0.25) (layer F.Cu) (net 15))
 (segment (start 152.1282 96.266) (end 152.1281 96.2659) (width 0.25) (layer F.Cu) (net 15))
 (segment (start 152.131 92.014) (end 152.131 92.964) (width 0.25) (layer F.Cu) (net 15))
 (segment (start 152.1308 92.964) (end 152.1308 93.914) (width 0.25) (layer F.Cu) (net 15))
 (segment (start 152.1308 92.014) (end 152.1308 92.964) (width 0.25) (layer F.Cu) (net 15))
 (segment (start 152.1308 92.964) (end 152.131 92.964) (width 0.25) (layer F.Cu) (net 15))
 (segment (start 150.1318 92.964) (end 149.014 92.964) (width 0.25) (layer F.Cu) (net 11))
 (segment (start 149.014 92.964) (end 148.59 92.54) (width 0.25) (layer F.Cu) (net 11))
 (segment (start 150.132 92.964) (end 150.1318 92.964) (width 0.25) (layer F.Cu) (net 11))
 (segment (start 146.804 106.332) (end 146.804 106.358) (width 0.25) (layer F.Cu) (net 12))
 (segment (start 146.804 106.358) (end 146.482 106.68) (width 0.25) (layer F.Cu) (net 12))
 (segment (start 146.482 106.68) (end 140.97 106.68) (width 0.25) (layer F.Cu) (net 12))
 (segment (start 146.804 106.274) (end 146.804 106.332) (width 0.25) (layer F.Cu) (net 12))
 (segment (start 146.804 106.121) (end 146.804 106.274) (width 0.25) (layer F.Cu) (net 12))
 (segment (start 146.804 106.096) (end 146.804 106.121) (width 0.25) (layer F.Cu) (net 12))
 (segment (start 146.804 106.274) (end 146.804 106.332) (width 0.25) (layer F.Cu) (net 12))
 (segment (start 146.804 106.121) (end 146.804 106.274) (width 0.25) (layer F.Cu) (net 12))
 (segment (start 135.128 103.716) (end 137.387 103.716) (width 0.25) (layer F.Cu) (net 12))
 (segment (start 137.387 103.716) (end 137.414 103.743) (width 0.25) (layer F.Cu) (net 12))
 (segment (start 137.414 103.743) (end 137.414 106.426) (width 0.25) (layer F.Cu) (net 12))
 (segment (start 137.414 106.426) (end 137.668 106.68) (width 0.25) (layer F.Cu) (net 12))
 (segment (start 137.668 106.68) (end 140.97 106.68) (width 0.25) (layer F.Cu) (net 12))
 (segment (start 140.97 106.68) (end 141.29 107) (width 0.25) (layer F.Cu) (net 12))
 (segment (start 141.29 107) (end 141.29 107.866) (width 0.25) (layer F.Cu) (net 12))
 (segment (start 146.804 106.274) (end 146.533 106.274) (width 0.25) (layer F.Cu) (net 12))
 (segment (start 149.004 107.94) (end 149.014 107.95) (width 0.25) (layer F.Cu) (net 13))
 (segment (start 149.004 106.096) (end 149.004 107.94) (width 0.25) (layer F.Cu) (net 13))
 (segment (start 149.004 107.94) (end 149.014 107.95) (width 0.25) (layer F.Cu) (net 13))
 (segment (start 143.19 107.866) (end 148.93 107.866) (width 0.25) (layer F.Cu) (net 13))
 (segment (start 148.93 107.866) (end 149.004 107.94) (width 0.25) (layer F.Cu) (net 13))
 (segment (start 143.274 107.95) (end 143.19 107.866) (width 0.25) (layer F.Cu) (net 13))
 (segment (start 149.004 107.94) (end 149.014 107.95) (width 0.25) (layer F.Cu) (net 13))
 (segment (start 149.004 107.94) (end 149.014 107.95) (width 0.5) (layer F.Cu) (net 13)))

